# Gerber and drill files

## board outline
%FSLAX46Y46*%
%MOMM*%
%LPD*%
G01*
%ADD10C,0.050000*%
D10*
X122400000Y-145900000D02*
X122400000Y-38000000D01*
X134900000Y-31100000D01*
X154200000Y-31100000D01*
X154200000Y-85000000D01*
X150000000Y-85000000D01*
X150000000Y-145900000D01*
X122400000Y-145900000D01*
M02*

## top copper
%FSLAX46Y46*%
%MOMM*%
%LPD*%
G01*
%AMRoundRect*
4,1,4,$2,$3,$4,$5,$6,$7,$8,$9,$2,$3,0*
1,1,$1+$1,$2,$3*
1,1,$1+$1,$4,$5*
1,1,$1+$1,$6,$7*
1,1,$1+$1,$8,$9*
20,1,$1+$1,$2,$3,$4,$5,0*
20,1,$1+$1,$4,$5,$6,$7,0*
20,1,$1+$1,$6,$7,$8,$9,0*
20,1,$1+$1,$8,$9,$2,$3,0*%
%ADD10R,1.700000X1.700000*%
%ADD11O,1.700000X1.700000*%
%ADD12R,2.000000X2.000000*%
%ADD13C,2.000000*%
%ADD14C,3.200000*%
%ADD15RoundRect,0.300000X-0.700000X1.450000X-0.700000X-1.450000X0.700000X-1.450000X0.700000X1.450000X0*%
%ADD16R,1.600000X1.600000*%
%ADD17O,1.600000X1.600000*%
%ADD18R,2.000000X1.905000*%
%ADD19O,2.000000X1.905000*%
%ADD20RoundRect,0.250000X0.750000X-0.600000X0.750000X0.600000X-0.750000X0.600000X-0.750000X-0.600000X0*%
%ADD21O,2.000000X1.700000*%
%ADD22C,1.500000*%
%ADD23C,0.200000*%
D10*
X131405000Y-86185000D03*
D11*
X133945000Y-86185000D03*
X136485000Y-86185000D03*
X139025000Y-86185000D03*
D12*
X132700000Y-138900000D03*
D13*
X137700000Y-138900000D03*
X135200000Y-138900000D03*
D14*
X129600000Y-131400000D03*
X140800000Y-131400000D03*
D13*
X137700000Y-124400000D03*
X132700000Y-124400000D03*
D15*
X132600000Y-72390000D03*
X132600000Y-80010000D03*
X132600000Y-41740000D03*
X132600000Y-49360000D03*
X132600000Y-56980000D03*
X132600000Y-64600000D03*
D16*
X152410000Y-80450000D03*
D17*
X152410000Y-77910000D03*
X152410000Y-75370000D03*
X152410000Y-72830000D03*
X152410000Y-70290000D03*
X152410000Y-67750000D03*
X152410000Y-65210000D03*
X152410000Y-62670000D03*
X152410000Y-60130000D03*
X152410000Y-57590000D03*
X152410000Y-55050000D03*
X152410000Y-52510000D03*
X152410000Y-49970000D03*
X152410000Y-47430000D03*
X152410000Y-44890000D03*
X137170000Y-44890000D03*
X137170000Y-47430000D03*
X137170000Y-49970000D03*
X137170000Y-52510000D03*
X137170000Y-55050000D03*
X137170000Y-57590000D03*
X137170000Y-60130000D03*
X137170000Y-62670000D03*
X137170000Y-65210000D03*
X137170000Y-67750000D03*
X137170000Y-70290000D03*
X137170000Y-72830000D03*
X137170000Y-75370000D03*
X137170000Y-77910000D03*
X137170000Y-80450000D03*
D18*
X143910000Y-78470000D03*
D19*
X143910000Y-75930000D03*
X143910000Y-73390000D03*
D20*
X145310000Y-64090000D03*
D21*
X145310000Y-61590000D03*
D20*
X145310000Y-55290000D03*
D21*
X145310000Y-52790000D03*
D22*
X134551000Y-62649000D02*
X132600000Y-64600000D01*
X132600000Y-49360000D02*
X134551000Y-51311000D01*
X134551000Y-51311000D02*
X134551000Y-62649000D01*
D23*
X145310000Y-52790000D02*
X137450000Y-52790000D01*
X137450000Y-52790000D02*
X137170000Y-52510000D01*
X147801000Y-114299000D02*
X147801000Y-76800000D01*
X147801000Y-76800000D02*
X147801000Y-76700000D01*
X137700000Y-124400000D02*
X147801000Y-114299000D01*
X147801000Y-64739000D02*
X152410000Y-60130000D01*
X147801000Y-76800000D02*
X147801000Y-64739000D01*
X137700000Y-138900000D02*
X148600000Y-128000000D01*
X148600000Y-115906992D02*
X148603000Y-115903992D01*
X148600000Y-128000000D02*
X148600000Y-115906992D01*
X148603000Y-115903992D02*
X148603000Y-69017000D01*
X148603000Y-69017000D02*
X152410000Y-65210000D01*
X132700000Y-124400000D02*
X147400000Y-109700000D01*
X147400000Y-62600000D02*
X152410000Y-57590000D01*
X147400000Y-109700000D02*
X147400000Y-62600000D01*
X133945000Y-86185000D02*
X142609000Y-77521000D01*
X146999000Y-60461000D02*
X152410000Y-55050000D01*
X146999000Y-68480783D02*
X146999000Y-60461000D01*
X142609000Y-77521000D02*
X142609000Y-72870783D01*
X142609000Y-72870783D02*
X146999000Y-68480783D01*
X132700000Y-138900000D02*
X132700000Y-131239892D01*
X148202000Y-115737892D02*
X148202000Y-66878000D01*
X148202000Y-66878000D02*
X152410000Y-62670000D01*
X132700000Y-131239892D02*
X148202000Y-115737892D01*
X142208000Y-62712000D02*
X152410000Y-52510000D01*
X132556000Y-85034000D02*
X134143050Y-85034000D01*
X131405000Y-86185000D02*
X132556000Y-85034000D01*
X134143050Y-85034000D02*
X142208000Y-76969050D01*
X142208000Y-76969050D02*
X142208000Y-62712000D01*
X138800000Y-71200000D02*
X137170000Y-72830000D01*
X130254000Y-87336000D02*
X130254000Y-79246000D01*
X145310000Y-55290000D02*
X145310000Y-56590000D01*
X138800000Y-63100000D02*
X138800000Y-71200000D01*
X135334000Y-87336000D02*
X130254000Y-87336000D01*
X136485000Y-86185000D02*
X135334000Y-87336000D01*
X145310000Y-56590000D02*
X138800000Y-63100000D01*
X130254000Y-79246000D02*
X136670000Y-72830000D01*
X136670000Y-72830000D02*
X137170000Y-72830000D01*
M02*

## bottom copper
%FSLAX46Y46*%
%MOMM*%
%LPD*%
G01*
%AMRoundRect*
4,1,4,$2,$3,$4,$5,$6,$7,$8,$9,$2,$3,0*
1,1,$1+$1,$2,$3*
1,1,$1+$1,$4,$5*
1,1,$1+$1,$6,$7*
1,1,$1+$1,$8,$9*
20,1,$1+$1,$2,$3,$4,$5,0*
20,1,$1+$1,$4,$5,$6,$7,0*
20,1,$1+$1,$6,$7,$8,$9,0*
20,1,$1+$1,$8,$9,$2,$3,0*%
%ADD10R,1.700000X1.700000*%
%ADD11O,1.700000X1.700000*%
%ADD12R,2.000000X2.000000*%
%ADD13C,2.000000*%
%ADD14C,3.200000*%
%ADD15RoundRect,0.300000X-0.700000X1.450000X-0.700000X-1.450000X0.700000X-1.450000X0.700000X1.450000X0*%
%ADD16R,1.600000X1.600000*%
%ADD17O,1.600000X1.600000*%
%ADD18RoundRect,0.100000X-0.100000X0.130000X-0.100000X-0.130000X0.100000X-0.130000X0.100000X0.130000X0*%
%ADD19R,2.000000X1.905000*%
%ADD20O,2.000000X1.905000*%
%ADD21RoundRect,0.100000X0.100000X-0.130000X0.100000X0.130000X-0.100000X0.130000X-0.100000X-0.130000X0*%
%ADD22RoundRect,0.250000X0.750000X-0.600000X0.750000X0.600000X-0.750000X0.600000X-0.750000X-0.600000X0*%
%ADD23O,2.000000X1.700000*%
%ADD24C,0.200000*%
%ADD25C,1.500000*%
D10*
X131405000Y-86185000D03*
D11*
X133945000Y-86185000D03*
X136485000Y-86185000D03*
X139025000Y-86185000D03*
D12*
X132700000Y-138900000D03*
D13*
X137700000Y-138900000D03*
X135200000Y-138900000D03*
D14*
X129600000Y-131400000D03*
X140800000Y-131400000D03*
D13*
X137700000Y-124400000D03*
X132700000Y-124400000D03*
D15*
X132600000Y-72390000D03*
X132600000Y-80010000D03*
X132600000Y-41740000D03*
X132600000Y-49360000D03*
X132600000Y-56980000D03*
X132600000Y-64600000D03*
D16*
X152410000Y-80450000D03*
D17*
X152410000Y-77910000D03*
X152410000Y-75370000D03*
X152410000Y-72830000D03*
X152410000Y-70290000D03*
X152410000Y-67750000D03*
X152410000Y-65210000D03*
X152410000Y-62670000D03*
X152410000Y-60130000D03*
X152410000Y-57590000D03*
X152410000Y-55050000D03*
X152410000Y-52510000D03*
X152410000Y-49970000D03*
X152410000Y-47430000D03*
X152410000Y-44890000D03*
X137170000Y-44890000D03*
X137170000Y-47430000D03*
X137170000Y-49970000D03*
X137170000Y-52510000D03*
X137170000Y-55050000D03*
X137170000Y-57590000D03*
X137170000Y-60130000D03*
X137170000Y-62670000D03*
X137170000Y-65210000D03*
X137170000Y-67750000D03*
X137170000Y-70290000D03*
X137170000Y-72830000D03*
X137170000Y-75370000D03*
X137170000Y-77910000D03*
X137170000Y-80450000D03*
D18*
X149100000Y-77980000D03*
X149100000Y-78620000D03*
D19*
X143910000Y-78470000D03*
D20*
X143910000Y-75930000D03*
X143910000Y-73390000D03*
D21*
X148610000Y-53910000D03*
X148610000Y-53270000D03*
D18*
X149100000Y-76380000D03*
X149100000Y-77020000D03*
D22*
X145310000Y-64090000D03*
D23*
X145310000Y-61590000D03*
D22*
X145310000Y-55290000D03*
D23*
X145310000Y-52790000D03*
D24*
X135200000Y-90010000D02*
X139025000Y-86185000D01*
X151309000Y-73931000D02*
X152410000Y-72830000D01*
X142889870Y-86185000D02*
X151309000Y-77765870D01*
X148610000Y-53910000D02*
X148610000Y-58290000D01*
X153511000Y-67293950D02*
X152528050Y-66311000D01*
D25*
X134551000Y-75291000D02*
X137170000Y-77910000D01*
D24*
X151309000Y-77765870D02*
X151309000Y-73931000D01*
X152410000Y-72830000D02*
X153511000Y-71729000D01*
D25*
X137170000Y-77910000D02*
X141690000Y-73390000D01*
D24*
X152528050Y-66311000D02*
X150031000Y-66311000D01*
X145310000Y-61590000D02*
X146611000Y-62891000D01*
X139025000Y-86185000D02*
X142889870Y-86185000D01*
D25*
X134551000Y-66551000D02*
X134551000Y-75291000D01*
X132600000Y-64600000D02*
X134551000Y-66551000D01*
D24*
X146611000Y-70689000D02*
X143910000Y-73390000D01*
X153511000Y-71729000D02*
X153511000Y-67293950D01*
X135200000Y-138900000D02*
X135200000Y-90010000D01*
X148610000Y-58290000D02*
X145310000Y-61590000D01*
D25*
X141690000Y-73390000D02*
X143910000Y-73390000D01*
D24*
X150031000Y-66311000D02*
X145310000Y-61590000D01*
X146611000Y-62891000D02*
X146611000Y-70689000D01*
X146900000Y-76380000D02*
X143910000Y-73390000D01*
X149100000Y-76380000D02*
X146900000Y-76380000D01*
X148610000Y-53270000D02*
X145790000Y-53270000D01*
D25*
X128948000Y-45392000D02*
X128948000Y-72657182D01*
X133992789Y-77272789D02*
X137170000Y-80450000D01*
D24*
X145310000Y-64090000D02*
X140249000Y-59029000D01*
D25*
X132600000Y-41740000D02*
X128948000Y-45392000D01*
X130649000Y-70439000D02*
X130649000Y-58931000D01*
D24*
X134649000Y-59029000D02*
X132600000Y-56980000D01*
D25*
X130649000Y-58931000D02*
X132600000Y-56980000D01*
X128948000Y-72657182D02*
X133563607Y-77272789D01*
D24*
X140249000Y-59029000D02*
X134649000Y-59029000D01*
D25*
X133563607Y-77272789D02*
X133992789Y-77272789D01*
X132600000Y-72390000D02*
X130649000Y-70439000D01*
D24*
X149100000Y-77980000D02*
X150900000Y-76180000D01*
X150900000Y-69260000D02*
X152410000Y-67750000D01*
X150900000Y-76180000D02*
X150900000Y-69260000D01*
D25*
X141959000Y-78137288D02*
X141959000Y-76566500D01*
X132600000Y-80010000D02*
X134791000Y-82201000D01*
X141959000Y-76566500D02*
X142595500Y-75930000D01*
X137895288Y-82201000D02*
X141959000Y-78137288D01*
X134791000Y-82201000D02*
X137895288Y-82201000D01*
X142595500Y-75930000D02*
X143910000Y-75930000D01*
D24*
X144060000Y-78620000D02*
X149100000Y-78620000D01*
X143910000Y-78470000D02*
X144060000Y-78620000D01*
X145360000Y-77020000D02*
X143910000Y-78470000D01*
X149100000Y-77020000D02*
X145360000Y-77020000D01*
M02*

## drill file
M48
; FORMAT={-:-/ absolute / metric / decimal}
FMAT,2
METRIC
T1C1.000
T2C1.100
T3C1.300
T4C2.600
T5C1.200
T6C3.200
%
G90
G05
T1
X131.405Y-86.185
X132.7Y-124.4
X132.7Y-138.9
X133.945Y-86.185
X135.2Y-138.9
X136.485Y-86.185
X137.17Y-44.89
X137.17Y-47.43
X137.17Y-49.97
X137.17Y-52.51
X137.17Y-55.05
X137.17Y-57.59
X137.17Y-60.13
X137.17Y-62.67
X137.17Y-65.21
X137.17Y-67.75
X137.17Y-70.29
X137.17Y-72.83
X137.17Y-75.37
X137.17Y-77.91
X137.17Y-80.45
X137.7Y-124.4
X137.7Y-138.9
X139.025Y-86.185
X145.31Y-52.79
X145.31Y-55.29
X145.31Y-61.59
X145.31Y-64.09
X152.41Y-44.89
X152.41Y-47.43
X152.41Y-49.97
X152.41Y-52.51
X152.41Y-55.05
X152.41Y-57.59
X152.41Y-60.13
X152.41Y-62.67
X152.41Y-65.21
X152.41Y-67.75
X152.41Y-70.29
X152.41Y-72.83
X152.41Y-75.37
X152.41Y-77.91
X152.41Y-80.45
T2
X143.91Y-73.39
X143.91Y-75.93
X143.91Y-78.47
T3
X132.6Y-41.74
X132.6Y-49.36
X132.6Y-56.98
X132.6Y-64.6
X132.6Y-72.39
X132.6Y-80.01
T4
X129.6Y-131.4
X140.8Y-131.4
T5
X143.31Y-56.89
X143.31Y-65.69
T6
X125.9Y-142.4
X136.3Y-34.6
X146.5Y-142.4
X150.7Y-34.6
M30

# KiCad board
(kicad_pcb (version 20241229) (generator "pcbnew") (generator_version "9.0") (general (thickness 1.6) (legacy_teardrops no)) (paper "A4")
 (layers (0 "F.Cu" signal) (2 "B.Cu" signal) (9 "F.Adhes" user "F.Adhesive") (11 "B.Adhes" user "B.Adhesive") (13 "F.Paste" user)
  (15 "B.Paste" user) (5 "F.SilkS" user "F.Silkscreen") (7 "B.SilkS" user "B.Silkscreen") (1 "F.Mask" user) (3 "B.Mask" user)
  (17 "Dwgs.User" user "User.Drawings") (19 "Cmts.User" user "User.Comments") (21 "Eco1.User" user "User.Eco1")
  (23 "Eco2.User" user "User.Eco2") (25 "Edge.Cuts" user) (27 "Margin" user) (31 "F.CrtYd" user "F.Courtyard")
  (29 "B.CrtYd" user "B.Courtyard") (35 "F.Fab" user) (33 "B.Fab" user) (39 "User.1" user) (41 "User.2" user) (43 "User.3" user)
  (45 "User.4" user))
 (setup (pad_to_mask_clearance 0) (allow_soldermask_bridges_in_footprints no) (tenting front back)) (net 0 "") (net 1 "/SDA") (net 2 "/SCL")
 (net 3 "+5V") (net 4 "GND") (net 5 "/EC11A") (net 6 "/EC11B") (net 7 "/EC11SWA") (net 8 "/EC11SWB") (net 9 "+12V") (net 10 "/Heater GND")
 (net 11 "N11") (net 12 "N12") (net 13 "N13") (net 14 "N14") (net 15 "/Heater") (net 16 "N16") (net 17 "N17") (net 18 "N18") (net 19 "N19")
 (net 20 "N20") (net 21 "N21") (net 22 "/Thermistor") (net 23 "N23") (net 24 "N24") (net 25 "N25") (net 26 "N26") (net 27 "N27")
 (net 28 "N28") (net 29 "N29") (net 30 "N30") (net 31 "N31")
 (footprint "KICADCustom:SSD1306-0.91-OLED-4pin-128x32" (layer "F.Cu") (at 129.215 122.685 90)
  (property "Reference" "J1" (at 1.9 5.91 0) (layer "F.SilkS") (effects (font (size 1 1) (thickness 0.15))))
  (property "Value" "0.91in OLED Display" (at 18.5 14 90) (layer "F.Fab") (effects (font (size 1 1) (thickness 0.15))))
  (pad "1" thru_hole rect (at 36.5 2.19 90) (size 1.7 1.7) (drill 1) (layers "*.Cu" "*.Mask") (remove_unused_layers no) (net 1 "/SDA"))
  (pad "2" thru_hole oval (at 36.5 4.73 90) (size 1.7 1.7) (drill 1) (layers "*.Cu" "*.Mask") (remove_unused_layers no) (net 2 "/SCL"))
  (pad "3" thru_hole oval (at 36.5 7.27 90) (size 1.7 1.7) (drill 1) (layers "*.Cu" "*.Mask") (remove_unused_layers no) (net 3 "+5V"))
  (pad "4" thru_hole oval (at 36.5 9.81 90) (size 1.7 1.7) (drill 1) (layers "*.Cu" "*.Mask") (remove_unused_layers no) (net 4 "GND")))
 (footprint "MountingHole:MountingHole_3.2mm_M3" (layer "F.Cu") (at 146.5 142.4)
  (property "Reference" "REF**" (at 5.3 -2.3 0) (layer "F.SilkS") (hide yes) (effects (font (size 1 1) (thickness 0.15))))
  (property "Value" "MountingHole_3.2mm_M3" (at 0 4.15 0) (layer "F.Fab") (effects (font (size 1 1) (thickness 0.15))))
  (pad "" np_thru_hole circle (at 0 0) (size 3.2 3.2) (drill 3.2) (layers "*.Cu" "*.Mask")))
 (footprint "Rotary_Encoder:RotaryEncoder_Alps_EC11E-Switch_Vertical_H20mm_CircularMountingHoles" (layer "F.Cu") (at 132.7 138.9 90)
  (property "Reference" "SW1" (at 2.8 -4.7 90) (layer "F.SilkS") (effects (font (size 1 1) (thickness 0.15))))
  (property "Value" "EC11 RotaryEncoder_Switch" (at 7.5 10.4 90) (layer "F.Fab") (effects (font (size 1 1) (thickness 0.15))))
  (pad "A" thru_hole rect (at 0 0 90) (size 2 2) (drill 1) (layers "*.Cu" "*.Mask") (remove_unused_layers no) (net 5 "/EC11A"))
  (pad "B" thru_hole circle (at 0 5 90) (size 2 2) (drill 1) (layers "*.Cu" "*.Mask") (remove_unused_layers no) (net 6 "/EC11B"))
  (pad "C" thru_hole circle (at 0 2.5 90) (size 2 2) (drill 1) (layers "*.Cu" "*.Mask") (remove_unused_layers no) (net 4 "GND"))
  (pad "MP" thru_hole circle (at 7.5 -3.1 90) (size 3.2 3.2) (drill 2.6) (layers "*.Cu" "*.Mask") (remove_unused_layers no))
  (pad "MP" thru_hole circle (at 7.5 8.1 90) (size 3.2 3.2) (drill 2.6) (layers "*.Cu" "*.Mask") (remove_unused_layers no))
  (pad "S1" thru_hole circle (at 14.5 5 90) (size 2 2) (drill 1) (layers "*.Cu" "*.Mask") (remove_unused_layers no) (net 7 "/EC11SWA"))
  (pad "S2" thru_hole circle (at 14.5 0 90) (size 2 2) (drill 1) (layers "*.Cu" "*.Mask") (remove_unused_layers no) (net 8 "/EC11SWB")))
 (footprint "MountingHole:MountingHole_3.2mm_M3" (layer "F.Cu") (at 136.3 34.6)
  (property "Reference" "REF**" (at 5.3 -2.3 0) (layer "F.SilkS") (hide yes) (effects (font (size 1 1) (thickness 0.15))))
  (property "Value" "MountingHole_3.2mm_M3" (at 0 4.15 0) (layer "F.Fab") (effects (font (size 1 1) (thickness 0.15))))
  (pad "" np_thru_hole circle (at 0 0) (size 3.2 3.2) (drill 3.2) (layers "*.Cu" "*.Mask")))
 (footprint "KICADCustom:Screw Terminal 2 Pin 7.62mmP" (layer "F.Cu") (at 132.6 72.39 -90)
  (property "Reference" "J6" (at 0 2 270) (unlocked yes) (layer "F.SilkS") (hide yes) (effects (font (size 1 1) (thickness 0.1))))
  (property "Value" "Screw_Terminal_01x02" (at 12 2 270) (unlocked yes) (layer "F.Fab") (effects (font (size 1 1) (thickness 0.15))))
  (pad "1" thru_hole roundrect (at 0 0 270) (size 3.5 2) (drill 1.3) (layers "*.Cu" "*.Mask") (remove_unused_layers no)
   (roundrect_rratio 0.15) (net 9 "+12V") (thermal_bridge_angle 45))
  (pad "2" thru_hole roundrect (at 7.62 0 270) (size 3.5 2) (drill 1.3) (layers "*.Cu" "*.Mask") (remove_unused_layers no)
   (roundrect_rratio 0.15) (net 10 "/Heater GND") (thermal_bridge_angle 45)))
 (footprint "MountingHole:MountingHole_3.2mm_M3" (layer "F.Cu") (at 150.7 34.6)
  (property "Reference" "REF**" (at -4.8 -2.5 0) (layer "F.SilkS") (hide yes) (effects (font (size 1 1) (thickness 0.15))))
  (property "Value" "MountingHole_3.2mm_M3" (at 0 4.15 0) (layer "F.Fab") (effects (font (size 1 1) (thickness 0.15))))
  (pad "" np_thru_hole circle (at 0 0) (size 3.2 3.2) (drill 3.2) (layers "*.Cu" "*.Mask")))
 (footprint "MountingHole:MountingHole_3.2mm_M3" (layer "F.Cu") (at 125.9 142.4)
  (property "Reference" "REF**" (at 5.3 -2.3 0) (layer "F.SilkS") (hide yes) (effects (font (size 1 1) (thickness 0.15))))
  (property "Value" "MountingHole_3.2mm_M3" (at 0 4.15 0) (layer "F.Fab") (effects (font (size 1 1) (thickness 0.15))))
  (pad "" np_thru_hole circle (at 0 0) (size 3.2 3.2) (drill 3.2) (layers "*.Cu" "*.Mask")))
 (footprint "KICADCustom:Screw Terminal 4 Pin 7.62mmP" (layer "F.Cu") (at 132.6 41.74 -90)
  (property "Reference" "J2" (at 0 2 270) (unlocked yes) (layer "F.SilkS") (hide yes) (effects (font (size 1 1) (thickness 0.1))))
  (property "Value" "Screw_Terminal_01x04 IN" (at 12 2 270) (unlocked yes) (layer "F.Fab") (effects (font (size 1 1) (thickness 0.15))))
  (pad "1" thru_hole roundrect (at 0 0 270) (size 3.5 2) (drill 1.3) (layers "*.Cu" "*.Mask") (remove_unused_layers no)
   (roundrect_rratio 0.15) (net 9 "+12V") (thermal_bridge_angle 45))
  (pad "2" thru_hole roundrect (at 7.62 0 270) (size 3.5 2) (drill 1.3) (layers "*.Cu" "*.Mask") (remove_unused_layers no)
   (roundrect_rratio 0.15) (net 4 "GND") (thermal_bridge_angle 45))
  (pad "3" thru_hole roundrect (at 15.24 0 270) (size 3.5 2) (drill 1.3) (layers "*.Cu" "*.Mask") (remove_unused_layers no)
   (roundrect_rratio 0.15) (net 9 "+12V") (thermal_bridge_angle 45))
  (pad "4" thru_hole roundrect (at 22.86 0 270) (size 3.5 2) (drill 1.3) (layers "*.Cu" "*.Mask") (remove_unused_layers no)
   (roundrect_rratio 0.15) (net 4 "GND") (thermal_bridge_angle 45)))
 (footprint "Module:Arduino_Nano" (layer "F.Cu") (at 152.41 80.45 180)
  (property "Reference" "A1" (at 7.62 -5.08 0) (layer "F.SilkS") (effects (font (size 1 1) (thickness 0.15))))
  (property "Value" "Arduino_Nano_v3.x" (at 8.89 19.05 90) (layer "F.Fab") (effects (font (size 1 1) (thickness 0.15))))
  (pad "1" thru_hole rect (at 0 0 180) (size 1.6 1.6) (drill 1) (layers "*.Cu" "*.Mask") (remove_unused_layers no) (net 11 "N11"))
  (pad "2" thru_hole oval (at 0 2.54 180) (size 1.6 1.6) (drill 1) (layers "*.Cu" "*.Mask") (remove_unused_layers no) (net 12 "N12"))
  (pad "3" thru_hole oval (at 0 5.08 180) (size 1.6 1.6) (drill 1) (layers "*.Cu" "*.Mask") (remove_unused_layers no) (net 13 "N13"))
  (pad "4" thru_hole oval (at 0 7.62 180) (size 1.6 1.6) (drill 1) (layers "*.Cu" "*.Mask") (remove_unused_layers no) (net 4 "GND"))
  (pad "5" thru_hole oval (at 0 10.16 180) (size 1.6 1.6) (drill 1) (layers "*.Cu" "*.Mask") (remove_unused_layers no) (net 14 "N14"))
  (pad "6" thru_hole oval (at 0 12.7 180) (size 1.6 1.6) (drill 1) (layers "*.Cu" "*.Mask") (remove_unused_layers no) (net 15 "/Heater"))
  (pad "7" thru_hole oval (at 0 15.24 180) (size 1.6 1.6) (drill 1) (layers "*.Cu" "*.Mask") (remove_unused_layers no) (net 6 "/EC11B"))
  (pad "8" thru_hole oval (at 0 17.78 180) (size 1.6 1.6) (drill 1) (layers "*.Cu" "*.Mask") (remove_unused_layers no) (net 5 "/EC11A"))
  (pad "9" thru_hole oval (at 0 20.32 180) (size 1.6 1.6) (drill 1) (layers "*.Cu" "*.Mask") (remove_unused_layers no) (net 7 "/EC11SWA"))
  (pad "10" thru_hole oval (at 0 22.86 180) (size 1.6 1.6) (drill 1) (layers "*.Cu" "*.Mask") (remove_unused_layers no) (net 8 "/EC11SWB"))
  (pad "11" thru_hole oval (at 0 25.4 180) (size 1.6 1.6) (drill 1) (layers "*.Cu" "*.Mask") (remove_unused_layers no) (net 2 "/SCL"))
  (pad "12" thru_hole oval (at 0 27.94 180) (size 1.6 1.6) (drill 1) (layers "*.Cu" "*.Mask") (remove_unused_layers no) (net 1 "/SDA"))
  (pad "13" thru_hole oval (at 0 30.48 180) (size 1.6 1.6) (drill 1) (layers "*.Cu" "*.Mask") (remove_unused_layers no) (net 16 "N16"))
  (pad "14" thru_hole oval (at 0 33.02 180) (size 1.6 1.6) (drill 1) (layers "*.Cu" "*.Mask") (remove_unused_layers no) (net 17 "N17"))
  (pad "15" thru_hole oval (at 0 35.56 180) (size 1.6 1.6) (drill 1) (layers "*.Cu" "*.Mask") (remove_unused_layers no) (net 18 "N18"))
  (pad "16" thru_hole oval (at 15.24 35.56 180) (size 1.6 1.6) (drill 1) (layers "*.Cu" "*.Mask") (remove_unused_layers no) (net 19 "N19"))
  (pad "17" thru_hole oval (at 15.24 33.02 180) (size 1.6 1.6) (drill 1) (layers "*.Cu" "*.Mask") (remove_unused_layers no) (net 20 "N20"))
  (pad "18" thru_hole oval (at 15.24 30.48 180) (size 1.6 1.6) (drill 1) (layers "*.Cu" "*.Mask") (remove_unused_layers no) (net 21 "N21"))
  (pad "19" thru_hole oval (at 15.24 27.94 180) (size 1.6 1.6) (drill 1) (layers "*.Cu" "*.Mask") (remove_unused_layers no)
   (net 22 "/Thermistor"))
  (pad "20" thru_hole oval (at 15.24 25.4 180) (size 1.6 1.6) (drill 1) (layers "*.Cu" "*.Mask") (remove_unused_layers no) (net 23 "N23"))
  (pad "21" thru_hole oval (at 15.24 22.86 180) (size 1.6 1.6) (drill 1) (layers "*.Cu" "*.Mask") (remove_unused_layers no) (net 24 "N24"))
  (pad "22" thru_hole oval (at 15.24 20.32 180) (size 1.6 1.6) (drill 1) (layers "*.Cu" "*.Mask") (remove_unused_layers no) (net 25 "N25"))
  (pad "23" thru_hole oval (at 15.24 17.78 180) (size 1.6 1.6) (drill 1) (layers "*.Cu" "*.Mask") (remove_unused_layers no) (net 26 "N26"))
  (pad "24" thru_hole oval (at 15.24 15.24 180) (size 1.6 1.6) (drill 1) (layers "*.Cu" "*.Mask") (remove_unused_layers no) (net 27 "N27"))
  (pad "25" thru_hole oval (at 15.24 12.7 180) (size 1.6 1.6) (drill 1) (layers "*.Cu" "*.Mask") (remove_unused_layers no) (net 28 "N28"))
  (pad "26" thru_hole oval (at 15.24 10.16 180) (size 1.6 1.6) (drill 1) (layers "*.Cu" "*.Mask") (remove_unused_layers no) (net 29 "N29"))
  (pad "27" thru_hole oval (at 15.24 7.62 180) (size 1.6 1.6) (drill 1) (layers "*.Cu" "*.Mask") (remove_unused_layers no) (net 3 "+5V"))
  (pad "28" thru_hole oval (at 15.24 5.08 180) (size 1.6 1.6) (drill 1) (layers "*.Cu" "*.Mask") (remove_unused_layers no) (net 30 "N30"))
  (pad "29" thru_hole oval (at 15.24 2.54 180) (size 1.6 1.6) (drill 1) (layers "*.Cu" "*.Mask") (remove_unused_layers no) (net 4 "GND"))
  (pad "30" thru_hole oval (at 15.24 0 180) (size 1.6 1.6) (drill 1) (layers "*.Cu" "*.Mask") (remove_unused_layers no) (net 9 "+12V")))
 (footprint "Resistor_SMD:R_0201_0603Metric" (layer "B.Cu") (at 149.1 78.3 -90)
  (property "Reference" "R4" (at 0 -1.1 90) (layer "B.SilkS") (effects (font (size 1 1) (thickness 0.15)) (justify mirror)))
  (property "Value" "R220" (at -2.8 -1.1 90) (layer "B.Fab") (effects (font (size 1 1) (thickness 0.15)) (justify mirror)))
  (pad "" smd roundrect (at -0.345 0 270) (size 0.318 0.36) (layers "B.Paste") (roundrect_rratio 0.25))
  (pad "" smd roundrect (at 0.345 0 270) (size 0.318 0.36) (layers "B.Paste") (roundrect_rratio 0.25))
  (pad "1" smd roundrect (at -0.32 0 270) (size 0.46 0.4) (layers "B.Cu" "B.Mask") (roundrect_rratio 0.25) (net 15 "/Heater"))
  (pad "2" smd roundrect (at 0.32 0 270) (size 0.46 0.4) (layers "B.Cu" "B.Mask") (roundrect_rratio 0.25) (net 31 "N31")))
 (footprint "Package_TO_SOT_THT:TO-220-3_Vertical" (layer "B.Cu") (at 143.91 78.47 90)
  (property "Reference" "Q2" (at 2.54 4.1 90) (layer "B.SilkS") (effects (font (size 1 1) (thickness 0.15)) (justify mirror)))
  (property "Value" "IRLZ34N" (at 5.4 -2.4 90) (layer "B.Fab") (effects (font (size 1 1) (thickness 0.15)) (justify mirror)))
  (pad "1" thru_hole rect (at 0 0 90) (size 1.905 2) (drill 1.1) (layers "*.Cu" "*.Mask") (remove_unused_layers no) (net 31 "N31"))
  (pad "2" thru_hole oval (at 2.54 0 90) (size 1.905 2) (drill 1.1) (layers "*.Cu" "*.Mask") (remove_unused_layers no)
   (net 10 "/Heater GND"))
  (pad "3" thru_hole oval (at 5.08 0 90) (size 1.905 2) (drill 1.1) (layers "*.Cu" "*.Mask") (remove_unused_layers no) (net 4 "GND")))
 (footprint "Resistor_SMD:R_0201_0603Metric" (layer "B.Cu") (at 148.61 53.59 90)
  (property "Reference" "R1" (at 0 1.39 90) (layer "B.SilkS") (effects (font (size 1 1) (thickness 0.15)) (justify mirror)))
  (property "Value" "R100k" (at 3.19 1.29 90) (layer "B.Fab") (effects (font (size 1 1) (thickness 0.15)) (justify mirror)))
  (pad "" smd roundrect (at -0.345 0 90) (size 0.318 0.36) (layers "B.Paste") (roundrect_rratio 0.25))
  (pad "" smd roundrect (at 0.345 0 90) (size 0.318 0.36) (layers "B.Paste") (roundrect_rratio 0.25))
  (pad "1" smd roundrect (at -0.32 0 90) (size 0.46 0.4) (layers "B.Cu" "B.Mask") (roundrect_rratio 0.25) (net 4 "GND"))
  (pad "2" smd roundrect (at 0.32 0 90) (size 0.46 0.4) (layers "B.Cu" "B.Mask") (roundrect_rratio 0.25) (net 22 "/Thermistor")))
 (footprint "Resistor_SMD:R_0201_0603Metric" (layer "B.Cu") (at 149.1 76.7 -90)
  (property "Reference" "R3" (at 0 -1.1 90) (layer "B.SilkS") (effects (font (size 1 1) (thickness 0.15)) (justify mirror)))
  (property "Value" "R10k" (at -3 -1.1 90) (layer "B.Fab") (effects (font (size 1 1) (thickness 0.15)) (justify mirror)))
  (pad "" smd roundrect (at -0.345 0 270) (size 0.318 0.36) (layers "B.Paste") (roundrect_rratio 0.25))
  (pad "" smd roundrect (at 0.345 0 270) (size 0.318 0.36) (layers "B.Paste") (roundrect_rratio 0.25))
  (pad "1" smd roundrect (at -0.32 0 270) (size 0.46 0.4) (layers "B.Cu" "B.Mask") (roundrect_rratio 0.25) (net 4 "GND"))
  (pad "2" smd roundrect (at 0.32 0 270) (size 0.46 0.4) (layers "B.Cu" "B.Mask") (roundrect_rratio 0.25) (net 31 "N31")))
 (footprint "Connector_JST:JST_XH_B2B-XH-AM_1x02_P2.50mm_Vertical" (layer "B.Cu") (at 145.31 64.09 90)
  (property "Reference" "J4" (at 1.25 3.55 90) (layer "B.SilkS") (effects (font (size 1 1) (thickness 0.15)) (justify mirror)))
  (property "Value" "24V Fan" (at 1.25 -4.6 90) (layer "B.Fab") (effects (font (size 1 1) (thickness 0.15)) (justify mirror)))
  (pad "" np_thru_hole circle (at -1.6 -2 90) (size 1.2 1.2) (drill 1.2) (layers "*.Cu" "*.Mask"))
  (pad "1" thru_hole roundrect (at 0 0 90) (size 1.7 2) (drill 1) (layers "*.Cu" "*.Mask") (remove_unused_layers no)
   (roundrect_rratio 0.147059) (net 9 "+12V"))
  (pad "2" thru_hole oval (at 2.5 0 90) (size 1.7 2) (drill 1) (layers "*.Cu" "*.Mask") (remove_unused_layers no) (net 4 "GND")))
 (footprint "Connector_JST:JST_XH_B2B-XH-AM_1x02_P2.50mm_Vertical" (layer "B.Cu") (at 145.31 55.29 90)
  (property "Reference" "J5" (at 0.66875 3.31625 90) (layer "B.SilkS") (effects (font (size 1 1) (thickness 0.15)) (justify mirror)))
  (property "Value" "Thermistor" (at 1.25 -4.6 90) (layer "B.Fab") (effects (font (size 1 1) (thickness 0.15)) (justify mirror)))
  (pad "" np_thru_hole circle (at -1.6 -2 90) (size 1.2 1.2) (drill 1.2) (layers "*.Cu" "*.Mask"))
  (pad "1" thru_hole roundrect (at 0 0 90) (size 1.7 2) (drill 1) (layers "*.Cu" "*.Mask") (remove_unused_layers no)
   (roundrect_rratio 0.147059) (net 3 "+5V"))
  (pad "2" thru_hole oval (at 2.5 0 90) (size 1.7 2) (drill 1) (layers "*.Cu" "*.Mask") (remove_unused_layers no) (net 22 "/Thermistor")))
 (gr_poly
  (pts (xy 122.4 145.9) (xy 122.4 38) (xy 134.9 31.1) (xy 154.2 31.1) (xy 154.2 85) (xy 150 85) (xy 150 145.9))
  (stroke (width 0.05) (type solid)) (fill no) (layer "Edge.Cuts"))
 (segment (start 134.551 62.649) (end 132.6 64.6) (width 1.5) (layer "F.Cu") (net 4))
 (segment (start 132.6 49.36) (end 134.551 51.311) (width 1.5) (layer "F.Cu") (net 4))
 (segment (start 134.551 51.311) (end 134.551 62.649) (width 1.5) (layer "F.Cu") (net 4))
 (segment (start 135.2 90.01) (end 139.025 86.185) (width 0.2) (layer "B.Cu") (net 4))
 (segment (start 151.309 73.931) (end 152.41 72.83) (width 0.2) (layer "B.Cu") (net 4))
 (segment (start 142.88987 86.185) (end 151.309 77.76587) (width 0.2) (layer "B.Cu") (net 4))
 (segment (start 148.61 53.91) (end 148.61 58.29) (width 0.2) (layer "B.Cu") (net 4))
 (segment (start 153.511 67.29395) (end 152.52805 66.311) (width 0.2) (layer "B.Cu") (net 4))
 (segment (start 134.551 75.291) (end 137.17 77.91) (width 1.5) (layer "B.Cu") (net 4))
 (segment (start 151.309 77.76587) (end 151.309 73.931) (width 0.2) (layer "B.Cu") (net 4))
 (segment (start 152.41 72.83) (end 153.511 71.729) (width 0.2) (layer "B.Cu") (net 4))
 (segment (start 137.17 77.91) (end 141.69 73.39) (width 1.5) (layer "B.Cu") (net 4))
 (segment (start 152.52805 66.311) (end 150.031 66.311) (width 0.2) (layer "B.Cu") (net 4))
 (segment (start 145.31 61.59) (end 146.611 62.891) (width 0.2) (layer "B.Cu") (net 4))
 (segment (start 139.025 86.185) (end 142.88987 86.185) (width 0.2) (layer "B.Cu") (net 4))
 (segment (start 134.551 66.551) (end 134.551 75.291) (width 1.5) (layer "B.Cu") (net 4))
 (segment (start 132.6 64.6) (end 134.551 66.551) (width 1.5) (layer "B.Cu") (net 4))
 (segment (start 146.611 70.689) (end 143.91 73.39) (width 0.2) (layer "B.Cu") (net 4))
 (segment (start 153.511 71.729) (end 153.511 67.29395) (width 0.2) (layer "B.Cu") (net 4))
 (segment (start 135.2 138.9) (end 135.2 90.01) (width 0.2) (layer "B.Cu") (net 4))
 (segment (start 148.61 58.29) (end 145.31 61.59) (width 0.2) (layer "B.Cu") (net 4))
 (segment (start 141.69 73.39) (end 143.91 73.39) (width 1.5) (layer "B.Cu") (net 4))
 (segment (start 150.031 66.311) (end 145.31 61.59) (width 0.2) (layer "B.Cu") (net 4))
 (segment (start 146.611 62.891) (end 146.611 70.689) (width 0.2) (layer "B.Cu") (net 4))
 (segment (start 146.9 76.38) (end 143.91 73.39) (width 0.2) (layer "B.Cu") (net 4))
 (segment (start 149.1 76.38) (end 146.9 76.38) (width 0.2) (layer "B.Cu") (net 4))
 (segment (start 145.31 52.79) (end 137.45 52.79) (width 0.2) (layer "F.Cu") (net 22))
 (segment (start 137.45 52.79) (end 137.17 52.51) (width 0.2) (layer "F.Cu") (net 22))
 (segment (start 148.61 53.27) (end 145.79 53.27) (width 0.2) (layer "B.Cu") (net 22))
 (segment (start 147.801 114.299) (end 147.801 76.8) (width 0.2) (layer "F.Cu") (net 7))
 (segment (start 147.801 76.8) (end 147.801 76.7) (width 0.2) (layer "F.Cu") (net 7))
 (segment (start 137.7 124.4) (end 147.801 114.299) (width 0.2) (layer "F.Cu") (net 7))
 (segment (start 147.801 64.739) (end 152.41 60.13) (width 0.2) (layer "F.Cu") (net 7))
 (segment (start 147.801 76.8) (end 147.801 64.739) (width 0.2) (layer "F.Cu") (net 7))
 (segment (start 137.7 138.9) (end 148.6 128) (width 0.2) (layer "F.Cu") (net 6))
 (segment (start 148.6 115.906992) (end 148.603 115.903992) (width 0.2) (layer "F.Cu") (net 6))
 (segment (start 148.6 128) (end 148.6 115.906992) (width 0.2) (layer "F.Cu") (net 6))
 (segment (start 148.603 115.903992) (end 148.603 69.017) (width 0.2) (layer "F.Cu") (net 6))
 (segment (start 148.603 69.017) (end 152.41 65.21) (width 0.2) (layer "F.Cu") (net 6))
 (segment (start 132.7 124.4) (end 147.4 109.7) (width 0.2) (layer "F.Cu") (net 8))
 (segment (start 147.4 62.6) (end 152.41 57.59) (width 0.2) (layer "F.Cu") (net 8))
 (segment (start 147.4 109.7) (end 147.4 62.6) (width 0.2) (layer "F.Cu") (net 8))
 (segment (start 128.948 45.392) (end 128.948 72.657182) (width 1.5) (layer "B.Cu") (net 9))
 (segment (start 133.992789 77.272789) (end 137.17 80.45) (width 1.5) (layer "B.Cu") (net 9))
 (segment (start 145.31 64.09) (end 140.249 59.029) (width 0.2) (layer "B.Cu") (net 9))
 (segment (start 132.6 41.74) (end 128.948 45.392) (width 1.5) (layer "B.Cu") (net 9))
 (segment (start 130.649 70.439) (end 130.649 58.931) (width 1.5) (layer "B.Cu") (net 9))
 (segment (start 134.649 59.029) (end 132.6 56.98) (width 0.2) (layer "B.Cu") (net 9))
 (segment (start 130.649 58.931) (end 132.6 56.98) (width 1.5) (layer "B.Cu") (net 9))
 (segment (start 128.948 72.657182) (end 133.563607 77.272789) (width 1.5) (layer "B.Cu") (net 9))
 (segment (start 140.249 59.029) (end 134.649 59.029) (width 0.2) (layer "B.Cu") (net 9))
 (segment (start 133.563607 77.272789) (end 133.992789 77.272789) (width 1.5) (layer "B.Cu") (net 9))
 (segment (start 132.6 72.39) (end 130.649 70.439) (width 1.5) (layer "B.Cu") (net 9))
 (segment (start 133.945 86.185) (end 142.609 77.521) (width 0.2) (layer "F.Cu") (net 2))
 (segment (start 146.999 60.461) (end 152.41 55.05) (width 0.2) (layer "F.Cu") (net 2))
 (segment (start 146.999 68.480783) (end 146.999 60.461) (width 0.2) (layer "F.Cu") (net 2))
 (segment (start 142.609 77.521) (end 142.609 72.870783) (width 0.2) (layer "F.Cu") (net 2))
 (segment (start 142.609 72.870783) (end 146.999 68.480783) (width 0.2) (layer "F.Cu") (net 2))
 (segment (start 132.7 138.9) (end 132.7 131.239892) (width 0.2) (layer "F.Cu") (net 5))
 (segment (start 148.202 115.737892) (end 148.202 66.878) (width 0.2) (layer "F.Cu") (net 5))
 (segment (start 148.202 66.878) (end 152.41 62.67) (width 0.2) (layer "F.Cu") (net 5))
 (segment (start 132.7 131.239892) (end 148.202 115.737892) (width 0.2) (layer "F.Cu") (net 5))
 (segment (start 149.1 77.98) (end 150.9 76.18) (width 0.2) (layer "B.Cu") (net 15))
 (segment (start 150.9 69.26) (end 152.41 67.75) (width 0.2) (layer "B.Cu") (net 15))
 (segment (start 150.9 76.18) (end 150.9 69.26) (width 0.2) (layer "B.Cu") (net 15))
 (segment (start 142.208 62.712) (end 152.41 52.51) (width 0.2) (layer "F.Cu") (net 1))
 (segment (start 132.556 85.034) (end 134.14305 85.034) (width 0.2) (layer "F.Cu") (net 1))
 (segment (start 131.405 86.185) (end 132.556 85.034) (width 0.2) (layer "F.Cu") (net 1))
 (segment (start 134.14305 85.034) (end 142.208 76.96905) (width 0.2) (layer "F.Cu") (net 1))
 (segment (start 142.208 76.96905) (end 142.208 62.712) (width 0.2) (layer "F.Cu") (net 1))
 (segment (start 138.8 71.2) (end 137.17 72.83) (width 0.2) (layer "F.Cu") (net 3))
 (segment (start 130.254 87.336) (end 130.254 79.246) (width 0.2) (layer "F.Cu") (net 3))
 (segment (start 145.31 55.29) (end 145.31 56.59) (width 0.2) (layer "F.Cu") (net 3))
 (segment (start 138.8 63.1) (end 138.8 71.2) (width 0.2) (layer "F.Cu") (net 3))
 (segment (start 135.334 87.336) (end 130.254 87.336) (width 0.2) (layer "F.Cu") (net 3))
 (segment (start 136.485 86.185) (end 135.334 87.336) (width 0.2) (layer "F.Cu") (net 3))
 (segment (start 145.31 56.59) (end 138.8 63.1) (width 0.2) (layer "F.Cu") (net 3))
 (segment (start 130.254 79.246) (end 136.67 72.83) (width 0.2) (layer "F.Cu") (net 3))
 (segment (start 136.67 72.83) (end 137.17 72.83) (width 0.2) (layer "F.Cu") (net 3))
 (segment (start 141.959 78.137288) (end 141.959 76.5665) (width 1.5) (layer "B.Cu") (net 10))
 (segment (start 132.6 80.01) (end 134.791 82.201) (width 1.5) (layer "B.Cu") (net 10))
 (segment (start 141.959 76.5665) (end 142.5955 75.93) (width 1.5) (layer "B.Cu") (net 10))
 (segment (start 137.895288 82.201) (end 141.959 78.137288) (width 1.5) (layer "B.Cu") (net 10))
 (segment (start 134.791 82.201) (end 137.895288 82.201) (width 1.5) (layer "B.Cu") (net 10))
 (segment (start 142.5955 75.93) (end 143.91 75.93) (width 1.5) (layer "B.Cu") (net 10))
 (segment (start 144.06 78.62) (end 149.1 78.62) (width 0.2) (layer "B.Cu") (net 31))
 (segment (start 143.91 78.47) (end 144.06 78.62) (width 0.2) (layer "B.Cu") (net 31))
 (segment (start 145.36 77.02) (end 143.91 78.47) (width 0.2) (layer "B.Cu") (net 31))
 (segment (start 149.1 77.02) (end 145.36 77.02) (width 0.2) (layer "B.Cu") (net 31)))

